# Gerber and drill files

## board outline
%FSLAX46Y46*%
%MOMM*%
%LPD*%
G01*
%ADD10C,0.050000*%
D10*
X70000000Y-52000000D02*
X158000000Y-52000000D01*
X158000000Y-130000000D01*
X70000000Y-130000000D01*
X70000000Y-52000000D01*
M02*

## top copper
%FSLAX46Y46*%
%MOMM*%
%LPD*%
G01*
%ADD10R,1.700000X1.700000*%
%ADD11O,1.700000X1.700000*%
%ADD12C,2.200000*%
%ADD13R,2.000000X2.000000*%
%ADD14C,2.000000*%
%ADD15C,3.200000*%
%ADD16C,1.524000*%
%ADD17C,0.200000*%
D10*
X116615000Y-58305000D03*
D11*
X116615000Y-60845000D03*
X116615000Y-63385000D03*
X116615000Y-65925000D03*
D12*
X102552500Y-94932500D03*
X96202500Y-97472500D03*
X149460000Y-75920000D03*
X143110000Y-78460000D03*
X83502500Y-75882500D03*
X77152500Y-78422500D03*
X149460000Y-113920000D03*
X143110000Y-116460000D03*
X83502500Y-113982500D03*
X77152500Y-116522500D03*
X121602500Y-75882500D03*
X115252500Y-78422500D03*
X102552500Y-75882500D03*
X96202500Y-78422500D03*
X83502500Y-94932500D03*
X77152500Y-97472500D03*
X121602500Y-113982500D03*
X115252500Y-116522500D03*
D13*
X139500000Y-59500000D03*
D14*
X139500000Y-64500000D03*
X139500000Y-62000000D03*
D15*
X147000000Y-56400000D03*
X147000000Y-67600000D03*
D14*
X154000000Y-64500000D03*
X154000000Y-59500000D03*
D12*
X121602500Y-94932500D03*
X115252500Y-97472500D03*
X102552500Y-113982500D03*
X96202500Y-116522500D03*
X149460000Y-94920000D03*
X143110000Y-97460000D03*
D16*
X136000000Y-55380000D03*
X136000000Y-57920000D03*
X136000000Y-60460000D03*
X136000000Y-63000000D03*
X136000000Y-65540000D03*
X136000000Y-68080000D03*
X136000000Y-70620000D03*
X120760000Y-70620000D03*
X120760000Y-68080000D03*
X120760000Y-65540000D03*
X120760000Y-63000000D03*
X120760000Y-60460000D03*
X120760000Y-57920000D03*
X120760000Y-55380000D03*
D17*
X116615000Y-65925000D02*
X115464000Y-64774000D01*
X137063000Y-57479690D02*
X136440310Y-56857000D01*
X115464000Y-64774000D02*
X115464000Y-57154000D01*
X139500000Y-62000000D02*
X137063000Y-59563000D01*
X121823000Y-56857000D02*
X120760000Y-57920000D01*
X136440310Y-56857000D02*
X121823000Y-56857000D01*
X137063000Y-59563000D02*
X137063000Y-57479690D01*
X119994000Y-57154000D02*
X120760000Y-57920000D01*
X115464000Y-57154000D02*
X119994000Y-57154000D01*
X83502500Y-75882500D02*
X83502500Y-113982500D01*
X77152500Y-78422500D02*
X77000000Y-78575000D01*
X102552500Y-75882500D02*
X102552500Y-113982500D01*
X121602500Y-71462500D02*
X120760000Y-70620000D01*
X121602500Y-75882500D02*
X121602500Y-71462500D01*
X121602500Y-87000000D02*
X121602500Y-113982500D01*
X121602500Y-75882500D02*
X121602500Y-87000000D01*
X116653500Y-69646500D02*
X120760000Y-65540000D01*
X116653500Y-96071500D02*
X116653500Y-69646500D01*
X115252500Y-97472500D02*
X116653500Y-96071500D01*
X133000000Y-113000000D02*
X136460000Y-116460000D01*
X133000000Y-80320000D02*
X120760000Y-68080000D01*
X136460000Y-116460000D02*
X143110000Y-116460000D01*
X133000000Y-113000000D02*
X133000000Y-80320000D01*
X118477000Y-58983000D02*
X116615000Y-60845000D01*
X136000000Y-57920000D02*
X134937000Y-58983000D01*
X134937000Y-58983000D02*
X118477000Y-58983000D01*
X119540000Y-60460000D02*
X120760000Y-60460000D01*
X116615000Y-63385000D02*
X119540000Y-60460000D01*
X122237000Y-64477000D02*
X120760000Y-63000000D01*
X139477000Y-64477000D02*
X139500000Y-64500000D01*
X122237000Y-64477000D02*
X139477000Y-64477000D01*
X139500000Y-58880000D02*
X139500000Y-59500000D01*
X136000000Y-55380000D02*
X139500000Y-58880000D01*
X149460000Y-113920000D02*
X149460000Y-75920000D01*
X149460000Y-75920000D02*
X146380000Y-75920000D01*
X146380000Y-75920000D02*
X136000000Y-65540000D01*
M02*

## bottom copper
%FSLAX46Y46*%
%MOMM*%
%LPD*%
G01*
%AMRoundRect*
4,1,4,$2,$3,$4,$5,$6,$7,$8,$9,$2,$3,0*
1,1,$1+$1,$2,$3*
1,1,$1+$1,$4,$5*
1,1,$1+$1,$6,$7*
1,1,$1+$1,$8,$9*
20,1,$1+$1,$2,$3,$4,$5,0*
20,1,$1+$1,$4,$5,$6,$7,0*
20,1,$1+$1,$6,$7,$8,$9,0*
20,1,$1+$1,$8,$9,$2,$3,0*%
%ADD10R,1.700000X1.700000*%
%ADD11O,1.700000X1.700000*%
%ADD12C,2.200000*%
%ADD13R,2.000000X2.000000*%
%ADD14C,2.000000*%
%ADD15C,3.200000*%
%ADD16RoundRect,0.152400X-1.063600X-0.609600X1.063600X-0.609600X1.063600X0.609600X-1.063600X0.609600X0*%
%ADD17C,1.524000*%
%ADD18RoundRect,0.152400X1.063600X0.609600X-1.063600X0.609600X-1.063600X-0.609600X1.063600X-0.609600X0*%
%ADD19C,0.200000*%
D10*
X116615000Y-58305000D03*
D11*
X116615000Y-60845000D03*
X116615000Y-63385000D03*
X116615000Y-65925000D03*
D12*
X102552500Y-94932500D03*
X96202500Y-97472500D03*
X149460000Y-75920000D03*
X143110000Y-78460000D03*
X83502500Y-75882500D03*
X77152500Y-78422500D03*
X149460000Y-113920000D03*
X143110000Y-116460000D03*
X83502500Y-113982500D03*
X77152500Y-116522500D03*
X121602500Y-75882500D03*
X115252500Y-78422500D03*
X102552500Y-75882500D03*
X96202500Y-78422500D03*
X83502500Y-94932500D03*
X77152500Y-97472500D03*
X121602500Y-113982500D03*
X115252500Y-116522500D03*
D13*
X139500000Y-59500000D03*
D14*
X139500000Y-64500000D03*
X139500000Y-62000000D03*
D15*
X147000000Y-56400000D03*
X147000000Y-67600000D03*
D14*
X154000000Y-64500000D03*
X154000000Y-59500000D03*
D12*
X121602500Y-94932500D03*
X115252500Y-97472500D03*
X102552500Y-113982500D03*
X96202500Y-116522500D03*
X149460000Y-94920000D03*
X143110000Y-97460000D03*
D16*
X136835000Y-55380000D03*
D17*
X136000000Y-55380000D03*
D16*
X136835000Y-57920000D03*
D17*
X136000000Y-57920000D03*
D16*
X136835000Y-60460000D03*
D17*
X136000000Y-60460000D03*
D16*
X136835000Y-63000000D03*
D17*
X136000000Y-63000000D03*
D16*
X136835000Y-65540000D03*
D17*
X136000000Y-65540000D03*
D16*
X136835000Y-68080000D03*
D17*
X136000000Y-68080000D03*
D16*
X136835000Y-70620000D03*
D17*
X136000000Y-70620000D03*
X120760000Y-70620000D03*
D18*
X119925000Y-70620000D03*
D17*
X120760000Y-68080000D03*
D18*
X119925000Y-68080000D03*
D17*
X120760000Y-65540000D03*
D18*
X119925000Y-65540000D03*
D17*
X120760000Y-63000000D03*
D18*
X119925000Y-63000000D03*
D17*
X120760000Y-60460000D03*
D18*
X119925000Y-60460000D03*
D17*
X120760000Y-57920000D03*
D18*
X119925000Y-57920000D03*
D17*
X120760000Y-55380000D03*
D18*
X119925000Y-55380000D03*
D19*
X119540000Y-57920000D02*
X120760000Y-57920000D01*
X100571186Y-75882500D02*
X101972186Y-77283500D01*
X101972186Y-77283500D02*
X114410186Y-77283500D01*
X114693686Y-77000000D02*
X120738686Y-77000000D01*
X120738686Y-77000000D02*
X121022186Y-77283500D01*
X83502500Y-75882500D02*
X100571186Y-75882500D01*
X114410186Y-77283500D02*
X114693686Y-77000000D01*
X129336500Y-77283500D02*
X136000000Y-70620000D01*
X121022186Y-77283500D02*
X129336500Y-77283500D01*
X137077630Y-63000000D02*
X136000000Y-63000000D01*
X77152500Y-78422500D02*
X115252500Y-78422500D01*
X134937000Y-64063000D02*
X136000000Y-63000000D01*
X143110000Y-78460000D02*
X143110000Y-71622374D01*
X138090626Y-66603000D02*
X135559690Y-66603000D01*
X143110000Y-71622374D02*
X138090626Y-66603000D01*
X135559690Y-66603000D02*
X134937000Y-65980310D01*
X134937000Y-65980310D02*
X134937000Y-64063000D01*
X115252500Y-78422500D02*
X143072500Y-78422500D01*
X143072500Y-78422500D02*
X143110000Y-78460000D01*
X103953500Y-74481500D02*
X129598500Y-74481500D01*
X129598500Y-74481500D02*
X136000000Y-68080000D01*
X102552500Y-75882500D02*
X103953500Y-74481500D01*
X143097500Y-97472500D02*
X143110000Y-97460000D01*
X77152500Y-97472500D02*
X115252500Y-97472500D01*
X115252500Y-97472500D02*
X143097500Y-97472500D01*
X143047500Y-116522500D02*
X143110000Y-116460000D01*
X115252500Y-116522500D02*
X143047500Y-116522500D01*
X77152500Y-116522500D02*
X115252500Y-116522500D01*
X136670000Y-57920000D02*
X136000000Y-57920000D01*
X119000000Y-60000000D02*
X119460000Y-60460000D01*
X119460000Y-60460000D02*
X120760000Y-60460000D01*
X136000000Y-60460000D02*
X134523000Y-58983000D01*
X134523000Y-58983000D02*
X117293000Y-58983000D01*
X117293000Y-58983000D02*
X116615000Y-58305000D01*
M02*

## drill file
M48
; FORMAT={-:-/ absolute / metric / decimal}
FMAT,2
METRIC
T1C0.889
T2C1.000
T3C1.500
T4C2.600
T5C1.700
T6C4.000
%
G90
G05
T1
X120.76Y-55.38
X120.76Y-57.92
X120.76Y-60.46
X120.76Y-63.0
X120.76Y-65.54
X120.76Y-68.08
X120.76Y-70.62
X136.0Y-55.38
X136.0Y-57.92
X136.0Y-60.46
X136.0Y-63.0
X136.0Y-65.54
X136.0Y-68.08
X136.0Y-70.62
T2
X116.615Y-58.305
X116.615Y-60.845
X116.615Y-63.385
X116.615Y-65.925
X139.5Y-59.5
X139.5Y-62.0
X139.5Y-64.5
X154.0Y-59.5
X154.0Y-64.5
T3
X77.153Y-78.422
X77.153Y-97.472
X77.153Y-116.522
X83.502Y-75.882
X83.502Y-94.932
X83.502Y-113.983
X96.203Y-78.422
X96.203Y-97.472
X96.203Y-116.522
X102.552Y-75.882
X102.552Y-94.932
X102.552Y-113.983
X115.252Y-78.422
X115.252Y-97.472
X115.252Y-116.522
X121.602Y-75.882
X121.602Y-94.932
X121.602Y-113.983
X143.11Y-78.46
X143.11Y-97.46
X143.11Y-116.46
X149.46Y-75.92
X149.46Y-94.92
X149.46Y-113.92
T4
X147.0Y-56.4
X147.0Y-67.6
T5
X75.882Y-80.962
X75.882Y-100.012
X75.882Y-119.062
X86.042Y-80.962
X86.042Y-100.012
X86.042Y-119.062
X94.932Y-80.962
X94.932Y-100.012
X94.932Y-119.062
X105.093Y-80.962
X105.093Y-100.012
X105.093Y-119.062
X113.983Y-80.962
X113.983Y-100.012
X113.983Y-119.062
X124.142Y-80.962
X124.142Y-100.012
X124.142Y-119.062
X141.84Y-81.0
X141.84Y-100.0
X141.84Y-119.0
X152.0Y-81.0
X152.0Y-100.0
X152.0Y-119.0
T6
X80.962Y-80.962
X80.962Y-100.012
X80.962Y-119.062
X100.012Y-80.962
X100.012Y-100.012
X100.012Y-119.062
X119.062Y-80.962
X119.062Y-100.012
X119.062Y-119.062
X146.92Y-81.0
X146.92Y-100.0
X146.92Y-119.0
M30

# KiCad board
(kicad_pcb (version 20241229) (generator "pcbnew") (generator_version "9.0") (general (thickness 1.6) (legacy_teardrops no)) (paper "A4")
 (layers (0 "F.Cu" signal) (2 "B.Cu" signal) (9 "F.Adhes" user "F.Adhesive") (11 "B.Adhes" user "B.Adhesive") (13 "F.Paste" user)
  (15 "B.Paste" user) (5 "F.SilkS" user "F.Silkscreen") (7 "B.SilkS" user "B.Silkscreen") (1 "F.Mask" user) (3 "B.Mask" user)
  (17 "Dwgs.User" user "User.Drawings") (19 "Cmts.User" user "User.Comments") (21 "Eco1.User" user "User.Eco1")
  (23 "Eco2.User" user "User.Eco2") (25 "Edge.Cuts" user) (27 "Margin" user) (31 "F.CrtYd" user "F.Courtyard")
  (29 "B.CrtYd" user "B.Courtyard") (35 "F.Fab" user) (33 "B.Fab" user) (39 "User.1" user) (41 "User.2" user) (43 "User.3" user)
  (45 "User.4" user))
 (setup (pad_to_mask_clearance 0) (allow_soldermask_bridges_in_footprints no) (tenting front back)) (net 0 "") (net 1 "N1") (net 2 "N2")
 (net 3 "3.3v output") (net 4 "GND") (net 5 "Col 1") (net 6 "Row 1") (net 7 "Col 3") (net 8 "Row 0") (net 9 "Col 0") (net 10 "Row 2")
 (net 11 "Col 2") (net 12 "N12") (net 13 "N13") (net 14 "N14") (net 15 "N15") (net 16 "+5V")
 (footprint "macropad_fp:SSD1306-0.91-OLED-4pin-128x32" (layer "F.Cu") (at 80.115 56.115)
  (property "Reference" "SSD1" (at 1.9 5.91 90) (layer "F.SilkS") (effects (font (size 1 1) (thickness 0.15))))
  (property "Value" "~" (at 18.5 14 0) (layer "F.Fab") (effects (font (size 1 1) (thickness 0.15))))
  (pad "1" thru_hole rect (at 36.5 2.19) (size 1.7 1.7) (drill 1) (layers "*.Cu" "*.Mask") (remove_unused_layers no) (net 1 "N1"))
  (pad "2" thru_hole oval (at 36.5 4.73) (size 1.7 1.7) (drill 1) (layers "*.Cu" "*.Mask") (remove_unused_layers no) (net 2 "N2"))
  (pad "3" thru_hole oval (at 36.5 7.27) (size 1.7 1.7) (drill 1) (layers "*.Cu" "*.Mask") (remove_unused_layers no) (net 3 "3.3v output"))
  (pad "4" thru_hole oval (at 36.5 9.81) (size 1.7 1.7) (drill 1) (layers "*.Cu" "*.Mask") (remove_unused_layers no) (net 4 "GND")))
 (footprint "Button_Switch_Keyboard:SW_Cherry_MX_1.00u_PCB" (layer "F.Cu") (at 102.5525 94.9325)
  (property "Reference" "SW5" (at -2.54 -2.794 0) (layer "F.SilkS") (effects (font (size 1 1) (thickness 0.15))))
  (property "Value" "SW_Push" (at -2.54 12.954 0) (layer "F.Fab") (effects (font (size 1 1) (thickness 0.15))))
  (pad "" np_thru_hole circle (at -7.62 5.08) (size 1.7 1.7) (drill 1.7) (layers "*.Cu" "*.Mask"))
  (pad "" np_thru_hole circle (at -2.54 5.08) (size 4 4) (drill 4) (layers "*.Cu" "*.Mask"))
  (pad "" np_thru_hole circle (at 2.54 5.08) (size 1.7 1.7) (drill 1.7) (layers "*.Cu" "*.Mask"))
  (pad "1" thru_hole circle (at 0 0) (size 2.2 2.2) (drill 1.5) (layers "*.Cu" "*.Mask") (remove_unused_layers no) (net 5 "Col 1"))
  (pad "2" thru_hole circle (at -6.35 2.54) (size 2.2 2.2) (drill 1.5) (layers "*.Cu" "*.Mask") (remove_unused_layers no) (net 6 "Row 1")))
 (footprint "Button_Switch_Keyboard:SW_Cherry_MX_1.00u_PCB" (layer "F.Cu") (at 149.46 75.92)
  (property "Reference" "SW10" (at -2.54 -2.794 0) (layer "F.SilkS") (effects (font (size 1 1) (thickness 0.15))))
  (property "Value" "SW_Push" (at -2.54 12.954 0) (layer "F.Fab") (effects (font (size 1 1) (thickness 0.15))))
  (pad "" np_thru_hole circle (at -7.62 5.08) (size 1.7 1.7) (drill 1.7) (layers "*.Cu" "*.Mask"))
  (pad "" np_thru_hole circle (at -2.54 5.08) (size 4 4) (drill 4) (layers "*.Cu" "*.Mask"))
  (pad "" np_thru_hole circle (at 2.54 5.08) (size 1.7 1.7) (drill 1.7) (layers "*.Cu" "*.Mask"))
  (pad "1" thru_hole circle (at 0 0) (size 2.2 2.2) (drill 1.5) (layers "*.Cu" "*.Mask") (remove_unused_layers no) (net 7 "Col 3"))
  (pad "2" thru_hole circle (at -6.35 2.54) (size 2.2 2.2) (drill 1.5) (layers "*.Cu" "*.Mask") (remove_unused_layers no) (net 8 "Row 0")))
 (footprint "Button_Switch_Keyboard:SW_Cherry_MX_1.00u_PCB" (layer "F.Cu") (at 83.5025 75.8825)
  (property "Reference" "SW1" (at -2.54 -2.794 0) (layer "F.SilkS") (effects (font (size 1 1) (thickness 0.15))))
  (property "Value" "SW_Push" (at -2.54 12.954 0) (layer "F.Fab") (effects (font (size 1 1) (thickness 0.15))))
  (pad "" np_thru_hole circle (at -7.62 5.08) (size 1.7 1.7) (drill 1.7) (layers "*.Cu" "*.Mask"))
  (pad "" np_thru_hole circle (at -2.54 5.08) (size 4 4) (drill 4) (layers "*.Cu" "*.Mask"))
  (pad "" np_thru_hole circle (at 2.54 5.08) (size 1.7 1.7) (drill 1.7) (layers "*.Cu" "*.Mask"))
  (pad "1" thru_hole circle (at 0 0) (size 2.2 2.2) (drill 1.5) (layers "*.Cu" "*.Mask") (remove_unused_layers no) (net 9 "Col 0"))
  (pad "2" thru_hole circle (at -6.35 2.54) (size 2.2 2.2) (drill 1.5) (layers "*.Cu" "*.Mask") (remove_unused_layers no) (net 8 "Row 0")))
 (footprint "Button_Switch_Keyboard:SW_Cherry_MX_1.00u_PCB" (layer "F.Cu") (at 149.46 113.92)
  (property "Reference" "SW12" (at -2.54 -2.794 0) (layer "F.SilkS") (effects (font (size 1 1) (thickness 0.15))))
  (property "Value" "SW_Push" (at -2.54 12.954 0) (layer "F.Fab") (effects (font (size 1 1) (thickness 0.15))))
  (pad "" np_thru_hole circle (at -7.62 5.08) (size 1.7 1.7) (drill 1.7) (layers "*.Cu" "*.Mask"))
  (pad "" np_thru_hole circle (at -2.54 5.08) (size 4 4) (drill 4) (layers "*.Cu" "*.Mask"))
  (pad "" np_thru_hole circle (at 2.54 5.08) (size 1.7 1.7) (drill 1.7) (layers "*.Cu" "*.Mask"))
  (pad "1" thru_hole circle (at 0 0) (size 2.2 2.2) (drill 1.5) (layers "*.Cu" "*.Mask") (remove_unused_layers no) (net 7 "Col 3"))
  (pad "2" thru_hole circle (at -6.35 2.54) (size 2.2 2.2) (drill 1.5) (layers "*.Cu" "*.Mask") (remove_unused_layers no) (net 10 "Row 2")))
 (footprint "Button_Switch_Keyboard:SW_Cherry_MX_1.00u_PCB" (layer "F.Cu") (at 83.5025 113.9825)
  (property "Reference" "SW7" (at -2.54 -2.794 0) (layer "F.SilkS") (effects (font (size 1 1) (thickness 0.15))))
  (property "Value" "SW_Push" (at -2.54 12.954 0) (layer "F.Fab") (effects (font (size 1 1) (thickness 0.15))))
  (pad "" np_thru_hole circle (at -7.62 5.08) (size 1.7 1.7) (drill 1.7) (layers "*.Cu" "*.Mask"))
  (pad "" np_thru_hole circle (at -2.54 5.08) (size 4 4) (drill 4) (layers "*.Cu" "*.Mask"))
  (pad "" np_thru_hole circle (at 2.54 5.08) (size 1.7 1.7) (drill 1.7) (layers "*.Cu" "*.Mask"))
  (pad "1" thru_hole circle (at 0 0) (size 2.2 2.2) (drill 1.5) (layers "*.Cu" "*.Mask") (remove_unused_layers no) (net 9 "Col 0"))
  (pad "2" thru_hole circle (at -6.35 2.54) (size 2.2 2.2) (drill 1.5) (layers "*.Cu" "*.Mask") (remove_unused_layers no) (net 10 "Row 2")))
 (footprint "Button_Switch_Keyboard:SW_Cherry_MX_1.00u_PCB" (layer "F.Cu") (at 121.6025 75.8825)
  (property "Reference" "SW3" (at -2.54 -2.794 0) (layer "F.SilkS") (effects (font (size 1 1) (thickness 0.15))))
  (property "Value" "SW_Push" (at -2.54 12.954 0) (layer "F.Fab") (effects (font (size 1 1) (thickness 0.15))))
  (pad "" np_thru_hole circle (at -7.62 5.08) (size 1.7 1.7) (drill 1.7) (layers "*.Cu" "*.Mask"))
  (pad "" np_thru_hole circle (at -2.54 5.08) (size 4 4) (drill 4) (layers "*.Cu" "*.Mask"))
  (pad "" np_thru_hole circle (at 2.54 5.08) (size 1.7 1.7) (drill 1.7) (layers "*.Cu" "*.Mask"))
  (pad "1" thru_hole circle (at 0 0) (size 2.2 2.2) (drill 1.5) (layers "*.Cu" "*.Mask") (remove_unused_layers no) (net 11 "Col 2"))
  (pad "2" thru_hole circle (at -6.35 2.54) (size 2.2 2.2) (drill 1.5) (layers "*.Cu" "*.Mask") (remove_unused_layers no) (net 8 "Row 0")))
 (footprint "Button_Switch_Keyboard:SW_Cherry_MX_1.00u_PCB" (layer "F.Cu") (at 102.5525 75.8825)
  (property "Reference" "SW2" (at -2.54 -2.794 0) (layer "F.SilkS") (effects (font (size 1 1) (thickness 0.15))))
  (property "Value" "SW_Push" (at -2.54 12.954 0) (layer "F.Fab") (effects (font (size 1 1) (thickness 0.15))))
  (pad "" np_thru_hole circle (at -7.62 5.08) (size 1.7 1.7) (drill 1.7) (layers "*.Cu" "*.Mask"))
  (pad "" np_thru_hole circle (at -2.54 5.08) (size 4 4) (drill 4) (layers "*.Cu" "*.Mask"))
  (pad "" np_thru_hole circle (at 2.54 5.08) (size 1.7 1.7) (drill 1.7) (layers "*.Cu" "*.Mask"))
  (pad "1" thru_hole circle (at 0 0) (size 2.2 2.2) (drill 1.5) (layers "*.Cu" "*.Mask") (remove_unused_layers no) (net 5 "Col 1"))
  (pad "2" thru_hole circle (at -6.35 2.54) (size 2.2 2.2) (drill 1.5) (layers "*.Cu" "*.Mask") (remove_unused_layers no) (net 8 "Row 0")))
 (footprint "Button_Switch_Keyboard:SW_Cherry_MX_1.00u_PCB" (layer "F.Cu") (at 83.5025 94.9325)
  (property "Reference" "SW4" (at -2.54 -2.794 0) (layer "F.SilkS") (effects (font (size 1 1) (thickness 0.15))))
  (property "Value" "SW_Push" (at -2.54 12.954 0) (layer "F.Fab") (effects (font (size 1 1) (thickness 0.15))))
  (pad "" np_thru_hole circle (at -7.62 5.08) (size 1.7 1.7) (drill 1.7) (layers "*.Cu" "*.Mask"))
  (pad "" np_thru_hole circle (at -2.54 5.08) (size 4 4) (drill 4) (layers "*.Cu" "*.Mask"))
  (pad "" np_thru_hole circle (at 2.54 5.08) (size 1.7 1.7) (drill 1.7) (layers "*.Cu" "*.Mask"))
  (pad "1" thru_hole circle (at 0 0) (size 2.2 2.2) (drill 1.5) (layers "*.Cu" "*.Mask") (remove_unused_layers no) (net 9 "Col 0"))
  (pad "2" thru_hole circle (at -6.35 2.54) (size 2.2 2.2) (drill 1.5) (layers "*.Cu" "*.Mask") (remove_unused_layers no) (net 6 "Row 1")))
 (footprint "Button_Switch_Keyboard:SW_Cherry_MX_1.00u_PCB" (layer "F.Cu") (at 121.6025 113.9825)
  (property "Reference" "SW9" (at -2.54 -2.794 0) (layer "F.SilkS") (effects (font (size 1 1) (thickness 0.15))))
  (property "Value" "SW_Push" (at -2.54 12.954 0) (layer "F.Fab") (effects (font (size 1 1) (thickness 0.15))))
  (pad "" np_thru_hole circle (at -7.62 5.08) (size 1.7 1.7) (drill 1.7) (layers "*.Cu" "*.Mask"))
  (pad "" np_thru_hole circle (at -2.54 5.08) (size 4 4) (drill 4) (layers "*.Cu" "*.Mask"))
  (pad "" np_thru_hole circle (at 2.54 5.08) (size 1.7 1.7) (drill 1.7) (layers "*.Cu" "*.Mask"))
  (pad "1" thru_hole circle (at 0 0) (size 2.2 2.2) (drill 1.5) (layers "*.Cu" "*.Mask") (remove_unused_layers no) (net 11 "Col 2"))
  (pad "2" thru_hole circle (at -6.35 2.54) (size 2.2 2.2) (drill 1.5) (layers "*.Cu" "*.Mask") (remove_unused_layers no) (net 10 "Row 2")))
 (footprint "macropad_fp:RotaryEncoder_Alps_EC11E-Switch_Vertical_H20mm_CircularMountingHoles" (layer "F.Cu") (at 139.5 59.5)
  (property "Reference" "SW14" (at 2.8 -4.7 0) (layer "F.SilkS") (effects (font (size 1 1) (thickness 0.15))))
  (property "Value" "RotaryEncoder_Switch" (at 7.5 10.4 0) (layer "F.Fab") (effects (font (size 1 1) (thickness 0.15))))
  (pad "A" thru_hole rect (at 0 0) (size 2 2) (drill 1) (layers "*.Cu" "*.Mask") (remove_unused_layers no) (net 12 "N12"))
  (pad "B" thru_hole circle (at 0 5) (size 2 2) (drill 1) (layers "*.Cu" "*.Mask") (remove_unused_layers no) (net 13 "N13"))
  (pad "C" thru_hole circle (at 0 2.5) (size 2 2) (drill 1) (layers "*.Cu" "*.Mask") (remove_unused_layers no) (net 4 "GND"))
  (pad "MP" thru_hole circle (at 7.5 -3.1) (size 3.2 3.2) (drill 2.6) (layers "*.Cu" "*.Mask") (remove_unused_layers no))
  (pad "MP" thru_hole circle (at 7.5 8.1) (size 3.2 3.2) (drill 2.6) (layers "*.Cu" "*.Mask") (remove_unused_layers no))
  (pad "S1" thru_hole circle (at 14.5 5) (size 2 2) (drill 1) (layers "*.Cu" "*.Mask") (remove_unused_layers no) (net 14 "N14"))
  (pad "S2" thru_hole circle (at 14.5 0) (size 2 2) (drill 1) (layers "*.Cu" "*.Mask") (remove_unused_layers no) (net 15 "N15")))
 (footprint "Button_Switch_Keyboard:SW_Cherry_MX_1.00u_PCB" (layer "F.Cu") (at 121.6025 94.9325)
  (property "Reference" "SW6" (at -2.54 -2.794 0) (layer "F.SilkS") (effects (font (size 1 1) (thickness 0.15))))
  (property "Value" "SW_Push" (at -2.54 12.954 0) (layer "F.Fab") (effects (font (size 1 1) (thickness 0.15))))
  (pad "" np_thru_hole circle (at -7.62 5.08) (size 1.7 1.7) (drill 1.7) (layers "*.Cu" "*.Mask"))
  (pad "" np_thru_hole circle (at -2.54 5.08) (size 4 4) (drill 4) (layers "*.Cu" "*.Mask"))
  (pad "" np_thru_hole circle (at 2.54 5.08) (size 1.7 1.7) (drill 1.7) (layers "*.Cu" "*.Mask"))
  (pad "1" thru_hole circle (at 0 0) (size 2.2 2.2) (drill 1.5) (layers "*.Cu" "*.Mask") (remove_unused_layers no) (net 11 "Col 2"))
  (pad "2" thru_hole circle (at -6.35 2.54) (size 2.2 2.2) (drill 1.5) (layers "*.Cu" "*.Mask") (remove_unused_layers no) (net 6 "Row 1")))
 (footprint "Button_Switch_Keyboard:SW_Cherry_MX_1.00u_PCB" (layer "F.Cu") (at 102.5525 113.9825)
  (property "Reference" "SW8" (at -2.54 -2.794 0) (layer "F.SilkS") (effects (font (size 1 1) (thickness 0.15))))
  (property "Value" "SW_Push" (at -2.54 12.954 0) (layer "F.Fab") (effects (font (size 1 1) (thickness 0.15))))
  (pad "" np_thru_hole circle (at -7.62 5.08) (size 1.7 1.7) (drill 1.7) (layers "*.Cu" "*.Mask"))
  (pad "" np_thru_hole circle (at -2.54 5.08) (size 4 4) (drill 4) (layers "*.Cu" "*.Mask"))
  (pad "" np_thru_hole circle (at 2.54 5.08) (size 1.7 1.7) (drill 1.7) (layers "*.Cu" "*.Mask"))
  (pad "1" thru_hole circle (at 0 0) (size 2.2 2.2) (drill 1.5) (layers "*.Cu" "*.Mask") (remove_unused_layers no) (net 5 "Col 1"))
  (pad "2" thru_hole circle (at -6.35 2.54) (size 2.2 2.2) (drill 1.5) (layers "*.Cu" "*.Mask") (remove_unused_layers no) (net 10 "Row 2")))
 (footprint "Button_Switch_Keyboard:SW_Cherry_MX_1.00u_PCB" (layer "F.Cu") (at 149.46 94.92)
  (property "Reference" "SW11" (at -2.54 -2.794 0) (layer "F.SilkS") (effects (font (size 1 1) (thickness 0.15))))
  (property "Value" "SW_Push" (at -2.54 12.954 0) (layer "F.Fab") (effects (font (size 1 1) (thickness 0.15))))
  (pad "" np_thru_hole circle (at -7.62 5.08) (size 1.7 1.7) (drill 1.7) (layers "*.Cu" "*.Mask"))
  (pad "" np_thru_hole circle (at -2.54 5.08) (size 4 4) (drill 4) (layers "*.Cu" "*.Mask"))
  (pad "" np_thru_hole circle (at 2.54 5.08) (size 1.7 1.7) (drill 1.7) (layers "*.Cu" "*.Mask"))
  (pad "1" thru_hole circle (at 0 0) (size 2.2 2.2) (drill 1.5) (layers "*.Cu" "*.Mask") (remove_unused_layers no) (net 7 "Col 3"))
  (pad "2" thru_hole circle (at -6.35 2.54) (size 2.2 2.2) (drill 1.5) (layers "*.Cu" "*.Mask") (remove_unused_layers no) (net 6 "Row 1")))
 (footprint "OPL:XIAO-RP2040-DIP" (layer "B.Cu") (at 128.38 63 180)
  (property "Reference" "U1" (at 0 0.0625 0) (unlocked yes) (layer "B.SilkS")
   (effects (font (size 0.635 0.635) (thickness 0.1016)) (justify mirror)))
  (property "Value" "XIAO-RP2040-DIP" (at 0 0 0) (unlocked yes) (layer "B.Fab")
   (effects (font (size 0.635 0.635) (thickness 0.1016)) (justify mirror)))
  (pad "1" smd roundrect (at -8.455 7.62) (size 2.432 1.524) (layers "B.Cu" "B.Mask") (roundrect_rratio 0.1) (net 12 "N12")
   (thermal_bridge_angle 45))
  (pad "1" thru_hole circle (at -7.62 7.62) (size 1.524 1.524) (drill 0.889) (layers "*.Cu" "*.Mask") (remove_unused_layers no)
   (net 12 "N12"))
  (pad "2" smd roundrect (at -8.455 5.08) (size 2.432 1.524) (layers "B.Cu" "B.Mask") (roundrect_rratio 0.1) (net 2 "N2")
   (thermal_bridge_angle 45))
  (pad "2" thru_hole circle (at -7.62 5.08) (size 1.524 1.524) (drill 0.889) (layers "*.Cu" "*.Mask") (remove_unused_layers no) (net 2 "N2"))
  (pad "3" smd roundrect (at -8.455 2.54) (size 2.432 1.524) (layers "B.Cu" "B.Mask") (roundrect_rratio 0.1) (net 1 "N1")
   (thermal_bridge_angle 45))
  (pad "3" thru_hole circle (at -7.62 2.54) (size 1.524 1.524) (drill 0.889) (layers "*.Cu" "*.Mask") (remove_unused_layers no) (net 1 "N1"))
  (pad "4" smd roundrect (at -8.455 0) (size 2.432 1.524) (layers "B.Cu" "B.Mask") (roundrect_rratio 0.1) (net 8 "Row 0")
   (thermal_bridge_angle 45))
  (pad "4" thru_hole circle (at -7.62 0) (size 1.524 1.524) (drill 0.889) (layers "*.Cu" "*.Mask") (remove_unused_layers no) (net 8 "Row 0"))
  (pad "5" smd roundrect (at -8.455 -2.54) (size 2.432 1.524) (layers "B.Cu" "B.Mask") (roundrect_rratio 0.1) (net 7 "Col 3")
   (thermal_bridge_angle 45))
  (pad "5" thru_hole circle (at -7.62 -2.54) (size 1.524 1.524) (drill 0.889) (layers "*.Cu" "*.Mask") (remove_unused_layers no)
   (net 7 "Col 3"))
  (pad "6" smd roundrect (at -8.455 -5.08) (size 2.432 1.524) (layers "B.Cu" "B.Mask") (roundrect_rratio 0.1) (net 5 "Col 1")
   (thermal_bridge_angle 45))
  (pad "6" thru_hole circle (at -7.62 -5.08) (size 1.524 1.524) (drill 0.889) (layers "*.Cu" "*.Mask") (remove_unused_layers no)
   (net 5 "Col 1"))
  (pad "7" smd roundrect (at -8.455 -7.62) (size 2.432 1.524) (layers "B.Cu" "B.Mask") (roundrect_rratio 0.1) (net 9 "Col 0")
   (thermal_bridge_angle 45))
  (pad "7" thru_hole circle (at -7.62 -7.62) (size 1.524 1.524) (drill 0.889) (layers "*.Cu" "*.Mask") (remove_unused_layers no)
   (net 9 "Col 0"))
  (pad "8" thru_hole circle (at 7.62 -7.62 180) (size 1.524 1.524) (drill 0.889) (layers "*.Cu" "*.Mask") (remove_unused_layers no)
   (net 11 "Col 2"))
  (pad "8" smd roundrect (at 8.455 -7.62 180) (size 2.432 1.524) (layers "B.Cu" "B.Mask") (roundrect_rratio 0.1) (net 11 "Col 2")
   (thermal_bridge_angle 45))
  (pad "9" thru_hole circle (at 7.62 -5.08 180) (size 1.524 1.524) (drill 0.889) (layers "*.Cu" "*.Mask") (remove_unused_layers no)
   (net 10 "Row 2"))
  (pad "9" smd roundrect (at 8.455 -5.08 180) (size 2.432 1.524) (layers "B.Cu" "B.Mask") (roundrect_rratio 0.1) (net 10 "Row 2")
   (thermal_bridge_angle 45))
  (pad "10" thru_hole circle (at 7.62 -2.54 180) (size 1.524 1.524) (drill 0.889) (layers "*.Cu" "*.Mask") (remove_unused_layers no)
   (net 6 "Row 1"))
  (pad "10" smd roundrect (at 8.455 -2.54 180) (size 2.432 1.524) (layers "B.Cu" "B.Mask") (roundrect_rratio 0.1) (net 6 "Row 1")
   (thermal_bridge_angle 45))
  (pad "11" thru_hole circle (at 7.62 0 180) (size 1.524 1.524) (drill 0.889) (layers "*.Cu" "*.Mask") (remove_unused_layers no)
   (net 13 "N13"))
  (pad "11" smd roundrect (at 8.455 0 180) (size 2.432 1.524) (layers "B.Cu" "B.Mask") (roundrect_rratio 0.1) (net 13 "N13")
   (thermal_bridge_angle 45))
  (pad "12" thru_hole circle (at 7.62 2.54 180) (size 1.524 1.524) (drill 0.889) (layers "*.Cu" "*.Mask") (remove_unused_layers no)
   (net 3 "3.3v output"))
  (pad "12" smd roundrect (at 8.455 2.54 180) (size 2.432 1.524) (layers "B.Cu" "B.Mask") (roundrect_rratio 0.1) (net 3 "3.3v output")
   (thermal_bridge_angle 45))
  (pad "13" thru_hole circle (at 7.62 5.08 180) (size 1.524 1.524) (drill 0.889) (layers "*.Cu" "*.Mask") (remove_unused_layers no)
   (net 4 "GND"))
  (pad "13" smd roundrect (at 8.455 5.08 180) (size 2.432 1.524) (layers "B.Cu" "B.Mask") (roundrect_rratio 0.1) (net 4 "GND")
   (thermal_bridge_angle 45))
  (pad "14" thru_hole circle (at 7.62 7.62 180) (size 1.524 1.524) (drill 0.889) (layers "*.Cu" "*.Mask") (remove_unused_layers no)
   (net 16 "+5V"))
  (pad "14" smd roundrect (at 8.455 7.62 180) (size 2.432 1.524) (layers "B.Cu" "B.Mask") (roundrect_rratio 0.1) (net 16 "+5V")
   (thermal_bridge_angle 45)))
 (gr_rect (start 70 52) (end 158 130) (stroke (width 0.05) (type solid)) (fill no) (layer "Edge.Cuts"))
 (segment (start 116.615 65.925) (end 115.464 64.774) (width 0.2) (layer "F.Cu") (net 4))
 (segment (start 137.063 57.47969) (end 136.44031 56.857) (width 0.2) (layer "F.Cu") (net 4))
 (segment (start 115.464 64.774) (end 115.464 57.154) (width 0.2) (layer "F.Cu") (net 4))
 (segment (start 139.5 62) (end 137.063 59.563) (width 0.2) (layer "F.Cu") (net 4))
 (segment (start 121.823 56.857) (end 120.76 57.92) (width 0.2) (layer "F.Cu") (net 4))
 (segment (start 136.44031 56.857) (end 121.823 56.857) (width 0.2) (layer "F.Cu") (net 4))
 (segment (start 137.063 59.563) (end 137.063 57.47969) (width 0.2) (layer "F.Cu") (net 4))
 (segment (start 119.994 57.154) (end 120.76 57.92) (width 0.2) (layer "F.Cu") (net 4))
 (segment (start 115.464 57.154) (end 119.994 57.154) (width 0.2) (layer "F.Cu") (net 4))
 (segment (start 119.54 57.92) (end 120.76 57.92) (width 0.2) (layer "B.Cu") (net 4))
 (segment (start 83.5025 75.8825) (end 83.5025 113.9825) (width 0.2) (layer "F.Cu") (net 9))
 (segment (start 100.571186 75.8825) (end 101.972186 77.2835) (width 0.2) (layer "B.Cu") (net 9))
 (segment (start 101.972186 77.2835) (end 114.410186 77.2835) (width 0.2) (layer "B.Cu") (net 9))
 (segment (start 114.693686 77) (end 120.738686 77) (width 0.2) (layer "B.Cu") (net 9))
 (segment (start 120.738686 77) (end 121.022186 77.2835) (width 0.2) (layer "B.Cu") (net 9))
 (segment (start 83.5025 75.8825) (end 100.571186 75.8825) (width 0.2) (layer "B.Cu") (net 9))
 (segment (start 114.410186 77.2835) (end 114.693686 77) (width 0.2) (layer "B.Cu") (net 9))
 (segment (start 129.3365 77.2835) (end 136 70.62) (width 0.2) (layer "B.Cu") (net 9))
 (segment (start 121.022186 77.2835) (end 129.3365 77.2835) (width 0.2) (layer "B.Cu") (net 9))
 (segment (start 77.1525 78.4225) (end 77 78.575) (width 0.2) (layer "F.Cu") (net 8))
 (segment (start 137.07763 63) (end 136 63) (width 0.2) (layer "B.Cu") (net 8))
 (segment (start 77.1525 78.4225) (end 115.2525 78.4225) (width 0.2) (layer "B.Cu") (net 8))
 (segment (start 134.937 64.063) (end 136 63) (width 0.2) (layer "B.Cu") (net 8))
 (segment (start 143.11 78.46) (end 143.11 71.622374) (width 0.2) (layer "B.Cu") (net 8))
 (segment (start 138.090626 66.603) (end 135.55969 66.603) (width 0.2) (layer "B.Cu") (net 8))
 (segment (start 143.11 71.622374) (end 138.090626 66.603) (width 0.2) (layer "B.Cu") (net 8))
 (segment (start 135.55969 66.603) (end 134.937 65.98031) (width 0.2) (layer "B.Cu") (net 8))
 (segment (start 134.937 65.98031) (end 134.937 64.063) (width 0.2) (layer "B.Cu") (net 8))
 (segment (start 115.2525 78.4225) (end 143.0725 78.4225) (width 0.2) (layer "B.Cu") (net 8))
 (segment (start 143.0725 78.4225) (end 143.11 78.46) (width 0.2) (layer "B.Cu") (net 8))
 (segment (start 102.5525 75.8825) (end 102.5525 113.9825) (width 0.2) (layer "F.Cu") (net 5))
 (segment (start 103.9535 74.4815) (end 129.5985 74.4815) (width 0.2) (layer "B.Cu") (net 5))
 (segment (start 129.5985 74.4815) (end 136 68.08) (width 0.2) (layer "B.Cu") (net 5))
 (segment (start 102.5525 75.8825) (end 103.9535 74.4815) (width 0.2) (layer "B.Cu") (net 5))
 (segment (start 121.6025 71.4625) (end 120.76 70.62) (width 0.2) (layer "F.Cu") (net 11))
 (segment (start 121.6025 75.8825) (end 121.6025 71.4625) (width 0.2) (layer "F.Cu") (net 11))
 (segment (start 121.6025 87) (end 121.6025 113.9825) (width 0.2) (layer "F.Cu") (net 11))
 (segment (start 121.6025 75.8825) (end 121.6025 87) (width 0.2) (layer "F.Cu") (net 11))
 (segment (start 116.6535 69.6465) (end 120.76 65.54) (width 0.2) (layer "F.Cu") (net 6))
 (segment (start 116.6535 96.0715) (end 116.6535 69.6465) (width 0.2) (layer "F.Cu") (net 6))
 (segment (start 115.2525 97.4725) (end 116.6535 96.0715) (width 0.2) (layer "F.Cu") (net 6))
 (segment (start 143.0975 97.4725) (end 143.11 97.46) (width 0.2) (layer "B.Cu") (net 6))
 (segment (start 77.1525 97.4725) (end 115.2525 97.4725) (width 0.2) (layer "B.Cu") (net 6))
 (segment (start 115.2525 97.4725) (end 143.0975 97.4725) (width 0.2) (layer "B.Cu") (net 6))
 (segment (start 133 113) (end 136.46 116.46) (width 0.2) (layer "F.Cu") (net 10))
 (segment (start 133 80.32) (end 120.76 68.08) (width 0.2) (layer "F.Cu") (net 10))
 (segment (start 136.46 116.46) (end 143.11 116.46) (width 0.2) (layer "F.Cu") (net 10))
 (segment (start 133 113) (end 133 80.32) (width 0.2) (layer "F.Cu") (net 10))
 (segment (start 143.0475 116.5225) (end 143.11 116.46) (width 0.2) (layer "B.Cu") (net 10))
 (segment (start 115.2525 116.5225) (end 143.0475 116.5225) (width 0.2) (layer "B.Cu") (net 10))
 (segment (start 77.1525 116.5225) (end 115.2525 116.5225) (width 0.2) (layer "B.Cu") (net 10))
 (segment (start 118.477 58.983) (end 116.615 60.845) (width 0.2) (layer "F.Cu") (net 2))
 (segment (start 136 57.92) (end 134.937 58.983) (width 0.2) (layer "F.Cu") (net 2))
 (segment (start 134.937 58.983) (end 118.477 58.983) (width 0.2) (layer "F.Cu") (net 2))
 (segment (start 136.67 57.92) (end 136 57.92) (width 0.2) (layer "B.Cu") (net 2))
 (segment (start 119.54 60.46) (end 120.76 60.46) (width 0.2) (layer "F.Cu") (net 3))
 (segment (start 116.615 63.385) (end 119.54 60.46) (width 0.2) (layer "F.Cu") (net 3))
 (segment (start 119 60) (end 119.46 60.46) (width 0.2) (layer "B.Cu") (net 3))
 (segment (start 119.46 60.46) (end 120.76 60.46) (width 0.2) (layer "B.Cu") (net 3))
 (segment (start 136 60.46) (end 134.523 58.983) (width 0.2) (layer "B.Cu") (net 1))
 (segment (start 134.523 58.983) (end 117.293 58.983) (width 0.2) (layer "B.Cu") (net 1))
 (segment (start 117.293 58.983) (end 116.615 58.305) (width 0.2) (layer "B.Cu") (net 1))
 (segment (start 122.237 64.477) (end 120.76 63) (width 0.2) (layer "F.Cu") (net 13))
 (segment (start 139.477 64.477) (end 139.5 64.5) (width 0.2) (layer "F.Cu") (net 13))
 (segment (start 122.237 64.477) (end 139.477 64.477) (width 0.2) (layer "F.Cu") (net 13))
 (segment (start 139.5 58.88) (end 139.5 59.5) (width 0.2) (layer "F.Cu") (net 12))
 (segment (start 136 55.38) (end 139.5 58.88) (width 0.2) (layer "F.Cu") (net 12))
 (segment (start 149.46 113.92) (end 149.46 75.92) (width 0.2) (layer "F.Cu") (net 7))
 (segment (start 149.46 75.92) (end 146.38 75.92) (width 0.2) (layer "F.Cu") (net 7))
 (segment (start 146.38 75.92) (end 136 65.54) (width 0.2) (layer "F.Cu") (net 7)))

